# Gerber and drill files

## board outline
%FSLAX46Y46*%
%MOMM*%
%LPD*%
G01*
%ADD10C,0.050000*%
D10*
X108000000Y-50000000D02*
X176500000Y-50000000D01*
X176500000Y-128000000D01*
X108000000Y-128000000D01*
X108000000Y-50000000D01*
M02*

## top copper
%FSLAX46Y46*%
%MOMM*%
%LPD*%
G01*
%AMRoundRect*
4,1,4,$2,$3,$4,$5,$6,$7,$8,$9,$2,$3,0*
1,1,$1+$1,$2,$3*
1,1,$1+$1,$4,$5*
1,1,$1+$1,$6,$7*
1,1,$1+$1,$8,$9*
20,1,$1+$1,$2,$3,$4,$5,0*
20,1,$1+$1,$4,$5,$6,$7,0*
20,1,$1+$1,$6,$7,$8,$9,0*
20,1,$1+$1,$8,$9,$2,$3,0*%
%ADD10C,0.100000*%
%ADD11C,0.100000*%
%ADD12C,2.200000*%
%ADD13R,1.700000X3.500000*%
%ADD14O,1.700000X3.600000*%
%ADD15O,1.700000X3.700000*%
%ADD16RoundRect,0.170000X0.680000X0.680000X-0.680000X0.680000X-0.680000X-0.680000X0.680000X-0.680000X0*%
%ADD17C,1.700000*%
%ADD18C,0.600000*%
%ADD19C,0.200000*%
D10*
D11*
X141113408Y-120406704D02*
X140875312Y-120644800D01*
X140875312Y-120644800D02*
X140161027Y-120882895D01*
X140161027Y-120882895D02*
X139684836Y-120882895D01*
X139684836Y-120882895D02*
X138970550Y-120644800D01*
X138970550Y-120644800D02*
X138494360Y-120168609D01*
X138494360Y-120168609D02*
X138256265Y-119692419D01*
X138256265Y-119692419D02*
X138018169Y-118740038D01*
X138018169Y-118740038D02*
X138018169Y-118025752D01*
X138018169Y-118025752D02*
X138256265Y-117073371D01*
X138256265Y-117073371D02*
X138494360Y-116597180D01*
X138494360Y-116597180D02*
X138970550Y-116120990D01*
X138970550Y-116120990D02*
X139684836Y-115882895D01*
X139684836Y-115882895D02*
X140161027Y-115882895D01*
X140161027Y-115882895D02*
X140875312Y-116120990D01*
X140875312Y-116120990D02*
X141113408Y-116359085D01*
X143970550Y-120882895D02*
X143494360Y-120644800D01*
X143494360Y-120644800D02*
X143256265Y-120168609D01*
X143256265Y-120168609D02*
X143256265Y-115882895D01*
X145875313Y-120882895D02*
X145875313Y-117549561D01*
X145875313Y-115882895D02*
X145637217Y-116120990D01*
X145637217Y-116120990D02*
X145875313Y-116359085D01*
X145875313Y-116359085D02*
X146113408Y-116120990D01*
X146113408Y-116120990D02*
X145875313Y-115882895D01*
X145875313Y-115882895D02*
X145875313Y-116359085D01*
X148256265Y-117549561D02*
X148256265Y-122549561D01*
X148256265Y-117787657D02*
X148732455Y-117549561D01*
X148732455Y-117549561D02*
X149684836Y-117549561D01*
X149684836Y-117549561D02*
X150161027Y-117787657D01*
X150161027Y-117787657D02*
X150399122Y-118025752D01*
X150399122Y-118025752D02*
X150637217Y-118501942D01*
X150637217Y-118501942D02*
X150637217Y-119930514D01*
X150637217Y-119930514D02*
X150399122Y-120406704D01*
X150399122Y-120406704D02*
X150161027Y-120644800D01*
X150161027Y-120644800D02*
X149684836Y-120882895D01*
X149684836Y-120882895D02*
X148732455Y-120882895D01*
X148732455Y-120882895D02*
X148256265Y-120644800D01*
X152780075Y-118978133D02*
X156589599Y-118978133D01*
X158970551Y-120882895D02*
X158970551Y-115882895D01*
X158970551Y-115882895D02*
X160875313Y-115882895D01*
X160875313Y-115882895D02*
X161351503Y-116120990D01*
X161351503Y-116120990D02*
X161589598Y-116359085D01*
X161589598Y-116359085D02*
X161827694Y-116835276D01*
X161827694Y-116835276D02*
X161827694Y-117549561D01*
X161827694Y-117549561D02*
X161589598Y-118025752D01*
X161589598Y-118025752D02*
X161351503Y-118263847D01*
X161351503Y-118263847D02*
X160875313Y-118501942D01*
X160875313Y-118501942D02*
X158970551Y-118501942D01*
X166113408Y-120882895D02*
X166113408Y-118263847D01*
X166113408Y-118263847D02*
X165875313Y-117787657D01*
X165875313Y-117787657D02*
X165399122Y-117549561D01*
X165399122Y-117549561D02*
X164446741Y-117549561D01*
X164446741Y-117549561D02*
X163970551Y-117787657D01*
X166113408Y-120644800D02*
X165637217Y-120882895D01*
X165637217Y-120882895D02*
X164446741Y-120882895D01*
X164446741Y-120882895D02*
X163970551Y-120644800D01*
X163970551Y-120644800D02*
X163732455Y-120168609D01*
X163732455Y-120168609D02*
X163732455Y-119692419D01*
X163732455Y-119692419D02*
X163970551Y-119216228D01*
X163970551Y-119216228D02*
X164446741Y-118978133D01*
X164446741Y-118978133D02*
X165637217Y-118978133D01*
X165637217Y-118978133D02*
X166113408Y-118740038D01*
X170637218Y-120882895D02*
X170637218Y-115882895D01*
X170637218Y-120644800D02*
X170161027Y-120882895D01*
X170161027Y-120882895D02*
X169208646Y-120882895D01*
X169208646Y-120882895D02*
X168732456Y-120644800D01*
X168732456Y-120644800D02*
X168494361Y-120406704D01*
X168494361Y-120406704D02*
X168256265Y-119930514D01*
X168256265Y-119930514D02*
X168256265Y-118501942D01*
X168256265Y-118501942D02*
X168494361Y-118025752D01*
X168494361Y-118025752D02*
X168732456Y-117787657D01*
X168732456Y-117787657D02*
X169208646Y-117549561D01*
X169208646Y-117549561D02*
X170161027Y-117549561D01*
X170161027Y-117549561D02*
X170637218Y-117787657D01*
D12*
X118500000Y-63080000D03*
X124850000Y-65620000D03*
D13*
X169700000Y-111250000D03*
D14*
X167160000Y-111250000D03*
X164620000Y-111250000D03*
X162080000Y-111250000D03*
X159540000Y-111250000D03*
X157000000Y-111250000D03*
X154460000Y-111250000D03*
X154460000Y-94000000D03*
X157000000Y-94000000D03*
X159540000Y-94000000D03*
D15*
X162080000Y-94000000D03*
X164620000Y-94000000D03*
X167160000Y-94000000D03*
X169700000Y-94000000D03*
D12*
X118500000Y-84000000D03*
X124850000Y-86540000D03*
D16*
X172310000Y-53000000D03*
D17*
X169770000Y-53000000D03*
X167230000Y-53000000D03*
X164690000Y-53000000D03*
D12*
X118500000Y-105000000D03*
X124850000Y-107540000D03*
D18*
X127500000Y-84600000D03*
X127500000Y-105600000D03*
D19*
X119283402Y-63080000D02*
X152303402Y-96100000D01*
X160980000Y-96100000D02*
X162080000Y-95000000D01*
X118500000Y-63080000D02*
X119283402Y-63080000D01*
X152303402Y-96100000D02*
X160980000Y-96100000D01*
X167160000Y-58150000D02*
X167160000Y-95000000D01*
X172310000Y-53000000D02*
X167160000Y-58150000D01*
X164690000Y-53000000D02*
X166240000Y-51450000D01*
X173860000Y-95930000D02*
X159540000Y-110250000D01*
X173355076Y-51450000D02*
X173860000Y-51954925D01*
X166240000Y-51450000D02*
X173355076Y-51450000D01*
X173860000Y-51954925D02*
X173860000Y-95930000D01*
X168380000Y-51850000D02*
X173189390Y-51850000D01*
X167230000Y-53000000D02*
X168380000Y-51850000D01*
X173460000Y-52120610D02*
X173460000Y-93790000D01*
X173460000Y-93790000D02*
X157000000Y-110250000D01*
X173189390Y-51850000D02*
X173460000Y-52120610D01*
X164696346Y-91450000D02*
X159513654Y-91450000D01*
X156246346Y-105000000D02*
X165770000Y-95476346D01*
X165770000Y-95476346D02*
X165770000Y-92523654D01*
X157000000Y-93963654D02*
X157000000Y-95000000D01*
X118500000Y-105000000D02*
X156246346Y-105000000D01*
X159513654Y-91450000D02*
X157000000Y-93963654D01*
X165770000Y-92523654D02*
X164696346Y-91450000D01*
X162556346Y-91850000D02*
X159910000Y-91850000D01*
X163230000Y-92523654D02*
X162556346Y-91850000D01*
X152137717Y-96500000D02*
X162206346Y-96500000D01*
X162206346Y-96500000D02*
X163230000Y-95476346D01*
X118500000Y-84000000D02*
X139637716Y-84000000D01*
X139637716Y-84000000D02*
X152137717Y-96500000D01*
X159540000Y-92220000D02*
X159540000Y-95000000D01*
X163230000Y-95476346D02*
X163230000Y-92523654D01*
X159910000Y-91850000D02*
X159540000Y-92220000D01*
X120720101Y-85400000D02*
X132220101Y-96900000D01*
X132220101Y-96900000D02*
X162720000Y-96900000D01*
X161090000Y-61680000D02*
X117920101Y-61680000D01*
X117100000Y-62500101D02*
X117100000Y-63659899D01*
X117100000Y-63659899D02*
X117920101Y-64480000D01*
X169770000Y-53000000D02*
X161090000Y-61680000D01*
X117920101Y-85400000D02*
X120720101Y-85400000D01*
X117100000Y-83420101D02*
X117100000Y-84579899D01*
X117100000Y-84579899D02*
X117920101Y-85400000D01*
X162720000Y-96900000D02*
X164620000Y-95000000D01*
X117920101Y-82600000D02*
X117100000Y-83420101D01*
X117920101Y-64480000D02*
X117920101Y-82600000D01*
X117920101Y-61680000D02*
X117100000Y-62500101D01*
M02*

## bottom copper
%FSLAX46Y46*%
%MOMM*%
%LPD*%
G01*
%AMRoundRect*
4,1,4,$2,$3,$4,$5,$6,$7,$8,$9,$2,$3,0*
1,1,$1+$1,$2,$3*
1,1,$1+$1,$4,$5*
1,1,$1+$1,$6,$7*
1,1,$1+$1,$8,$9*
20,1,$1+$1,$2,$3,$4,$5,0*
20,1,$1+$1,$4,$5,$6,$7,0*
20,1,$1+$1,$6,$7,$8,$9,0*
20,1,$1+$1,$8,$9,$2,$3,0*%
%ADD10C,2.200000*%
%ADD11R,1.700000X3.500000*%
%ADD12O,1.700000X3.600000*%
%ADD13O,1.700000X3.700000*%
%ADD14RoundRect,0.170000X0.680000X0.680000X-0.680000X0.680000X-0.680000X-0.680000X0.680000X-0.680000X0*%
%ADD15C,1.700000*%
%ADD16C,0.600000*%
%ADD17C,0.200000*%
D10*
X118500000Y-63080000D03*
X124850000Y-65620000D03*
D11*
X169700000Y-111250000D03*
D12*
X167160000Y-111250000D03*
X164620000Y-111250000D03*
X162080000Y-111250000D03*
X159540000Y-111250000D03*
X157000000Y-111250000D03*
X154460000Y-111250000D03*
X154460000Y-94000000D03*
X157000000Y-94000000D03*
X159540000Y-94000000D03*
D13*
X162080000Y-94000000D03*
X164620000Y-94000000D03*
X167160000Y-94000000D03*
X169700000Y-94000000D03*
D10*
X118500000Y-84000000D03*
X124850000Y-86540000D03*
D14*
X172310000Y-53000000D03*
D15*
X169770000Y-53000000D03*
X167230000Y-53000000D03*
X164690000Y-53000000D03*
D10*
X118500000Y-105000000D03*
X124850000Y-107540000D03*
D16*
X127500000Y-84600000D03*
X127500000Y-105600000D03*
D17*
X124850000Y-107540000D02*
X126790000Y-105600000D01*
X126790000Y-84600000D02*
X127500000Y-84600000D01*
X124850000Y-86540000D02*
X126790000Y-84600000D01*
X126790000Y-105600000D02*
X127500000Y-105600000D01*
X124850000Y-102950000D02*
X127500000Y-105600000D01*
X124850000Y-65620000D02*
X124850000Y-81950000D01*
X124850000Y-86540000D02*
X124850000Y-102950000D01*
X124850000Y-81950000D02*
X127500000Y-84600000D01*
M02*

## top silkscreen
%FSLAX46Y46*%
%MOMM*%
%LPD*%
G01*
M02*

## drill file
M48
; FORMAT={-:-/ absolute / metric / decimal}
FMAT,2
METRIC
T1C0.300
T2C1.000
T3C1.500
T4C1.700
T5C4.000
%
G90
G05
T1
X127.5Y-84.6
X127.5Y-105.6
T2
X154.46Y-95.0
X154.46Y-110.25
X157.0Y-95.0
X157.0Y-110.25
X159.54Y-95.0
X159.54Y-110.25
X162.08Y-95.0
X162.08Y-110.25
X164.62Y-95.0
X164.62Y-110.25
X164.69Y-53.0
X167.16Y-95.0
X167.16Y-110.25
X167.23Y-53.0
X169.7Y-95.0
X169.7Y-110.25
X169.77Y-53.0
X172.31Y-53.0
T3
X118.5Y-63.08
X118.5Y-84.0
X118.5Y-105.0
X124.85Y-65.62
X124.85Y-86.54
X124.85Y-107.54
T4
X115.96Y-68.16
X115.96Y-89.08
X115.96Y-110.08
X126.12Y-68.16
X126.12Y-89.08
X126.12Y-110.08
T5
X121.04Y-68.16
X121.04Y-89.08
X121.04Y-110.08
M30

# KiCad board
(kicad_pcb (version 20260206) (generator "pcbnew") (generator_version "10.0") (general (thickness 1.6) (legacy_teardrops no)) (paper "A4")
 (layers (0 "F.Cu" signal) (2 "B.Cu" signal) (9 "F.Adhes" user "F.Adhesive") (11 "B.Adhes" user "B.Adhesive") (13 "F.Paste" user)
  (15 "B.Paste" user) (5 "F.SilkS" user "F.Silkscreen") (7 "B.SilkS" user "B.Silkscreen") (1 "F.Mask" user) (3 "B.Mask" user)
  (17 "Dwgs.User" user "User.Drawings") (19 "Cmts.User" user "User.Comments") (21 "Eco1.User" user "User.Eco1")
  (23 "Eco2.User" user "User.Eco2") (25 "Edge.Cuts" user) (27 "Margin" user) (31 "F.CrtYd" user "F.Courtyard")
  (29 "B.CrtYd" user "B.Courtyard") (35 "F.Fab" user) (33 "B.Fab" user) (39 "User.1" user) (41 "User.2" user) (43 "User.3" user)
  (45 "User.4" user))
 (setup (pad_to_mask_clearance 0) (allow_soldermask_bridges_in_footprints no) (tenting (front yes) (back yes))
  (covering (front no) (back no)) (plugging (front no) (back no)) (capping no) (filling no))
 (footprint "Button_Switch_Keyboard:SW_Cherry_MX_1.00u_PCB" (layer "B.Cu") (at 118.5 63.08 180)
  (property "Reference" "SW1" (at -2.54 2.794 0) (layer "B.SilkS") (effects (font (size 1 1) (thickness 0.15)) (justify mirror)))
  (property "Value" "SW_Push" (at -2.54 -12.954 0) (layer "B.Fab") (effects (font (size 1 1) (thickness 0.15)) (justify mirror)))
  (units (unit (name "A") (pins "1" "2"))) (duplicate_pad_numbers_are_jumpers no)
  (pad "" np_thru_hole circle (at -7.62 -5.08 180) (size 1.7 1.7) (drill 1.7) (layers "*.Cu" "*.Mask"))
  (pad "" np_thru_hole circle (at -2.54 -5.08 180) (size 4 4) (drill 4) (layers "*.Cu" "*.Mask"))
  (pad "" np_thru_hole circle (at 2.54 -5.08 180) (size 1.7 1.7) (drill 1.7) (layers "*.Cu" "*.Mask"))
  (pad "1" thru_hole circle (at 0 0 180) (size 2.2 2.2) (drill 1.5) (layers "*.Cu" "*.Mask") (remove_unused_layers no)
   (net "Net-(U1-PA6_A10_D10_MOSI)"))
  (pad "2" thru_hole circle (at -6.35 -2.54 180) (size 2.2 2.2) (drill 1.5) (layers "*.Cu" "*.Mask") (remove_unused_layers no) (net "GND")))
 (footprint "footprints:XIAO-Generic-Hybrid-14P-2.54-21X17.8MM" (layer "B.Cu") (at 162.08 102.625 90)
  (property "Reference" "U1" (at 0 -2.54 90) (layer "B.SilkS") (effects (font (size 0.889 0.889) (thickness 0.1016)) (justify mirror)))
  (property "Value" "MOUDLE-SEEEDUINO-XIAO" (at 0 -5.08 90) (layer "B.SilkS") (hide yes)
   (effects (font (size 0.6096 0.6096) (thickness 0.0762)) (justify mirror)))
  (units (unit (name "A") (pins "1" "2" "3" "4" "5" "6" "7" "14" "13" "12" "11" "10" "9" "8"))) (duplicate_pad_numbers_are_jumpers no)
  (pad "1" thru_hole rect (at -7.625 7.62 90) (size 3.5 1.7) (drill 1 (offset -1 0)) (layers "*.Cu" "*.Mask") (remove_unused_layers no)
   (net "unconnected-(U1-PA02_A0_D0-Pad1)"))
  (pad "2" thru_hole oval (at -7.625 5.08 90) (size 3.6 1.7) (drill 1 (offset -1 0)) (layers "*.Cu" "*.Mask") (remove_unused_layers no)
   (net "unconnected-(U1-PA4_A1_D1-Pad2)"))
  (pad "3" thru_hole oval (at -7.625 2.54 90) (size 3.6 1.7) (drill 1 (offset -1 0)) (layers "*.Cu" "*.Mask") (remove_unused_layers no)
   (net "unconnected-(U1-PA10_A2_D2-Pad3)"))
  (pad "4" thru_hole oval (at -7.625 0 90) (size 3.6 1.7) (drill 1 (offset -1 0)) (layers "*.Cu" "*.Mask") (remove_unused_layers no)
   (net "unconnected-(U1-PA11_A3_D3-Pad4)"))
  (pad "5" thru_hole oval (at -7.625 -2.54 90) (size 3.6 1.7) (drill 1 (offset -1 0)) (layers "*.Cu" "*.Mask") (remove_unused_layers no)
   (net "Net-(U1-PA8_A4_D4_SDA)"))
  (pad "6" thru_hole oval (at -7.625 -5.08 270) (size 3.6 1.7) (drill 1 (offset 1 0)) (layers "*.Cu" "*.Mask") (remove_unused_layers no)
   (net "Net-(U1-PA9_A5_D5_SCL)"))
  (pad "7" thru_hole oval (at -7.625 -7.62 90) (size 3.6 1.7) (drill 1 (offset -1 0)) (layers "*.Cu" "*.Mask") (remove_unused_layers no)
   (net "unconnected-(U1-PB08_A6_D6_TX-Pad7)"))
  (pad "8" thru_hole oval (at 7.625 -7.62 90) (size 3.6 1.7) (drill 1 (offset 1 0)) (layers "*.Cu" "*.Mask") (remove_unused_layers no)
   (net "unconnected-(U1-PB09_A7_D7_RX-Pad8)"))
  (pad "9" thru_hole oval (at 7.625 -5.08 90) (size 3.6 1.7) (drill 1 (offset 1 0)) (layers "*.Cu" "*.Mask") (remove_unused_layers no)
   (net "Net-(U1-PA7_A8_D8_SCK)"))
  (pad "10" thru_hole oval (at 7.625 -2.54 90) (size 3.6 1.7) (drill 1 (offset 1 0)) (layers "*.Cu" "*.Mask") (remove_unused_layers no)
   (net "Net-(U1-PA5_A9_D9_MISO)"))
  (pad "11" thru_hole oval (at 7.625 0 90) (size 3.7 1.7) (drill 1 (offset 1 0)) (layers "*.Cu" "*.Mask") (remove_unused_layers no)
   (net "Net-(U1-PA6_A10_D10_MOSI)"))
  (pad "12" thru_hole oval (at 7.625 2.54 90) (size 3.7 1.7) (drill 1 (offset 1 0)) (layers "*.Cu" "*.Mask") (remove_unused_layers no)
   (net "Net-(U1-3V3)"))
  (pad "13" thru_hole oval (at 7.625 5.08 90) (size 3.7 1.7) (drill 1 (offset 1 0)) (layers "*.Cu" "*.Mask") (remove_unused_layers no)
   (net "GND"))
  (pad "14" thru_hole oval (at 7.625 7.62 90) (size 3.7 1.7) (drill 1 (offset 1 0)) (layers "*.Cu" "*.Mask") (remove_unused_layers no)
   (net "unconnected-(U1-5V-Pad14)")))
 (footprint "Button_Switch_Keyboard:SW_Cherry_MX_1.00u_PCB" (layer "B.Cu") (at 118.5 84 180)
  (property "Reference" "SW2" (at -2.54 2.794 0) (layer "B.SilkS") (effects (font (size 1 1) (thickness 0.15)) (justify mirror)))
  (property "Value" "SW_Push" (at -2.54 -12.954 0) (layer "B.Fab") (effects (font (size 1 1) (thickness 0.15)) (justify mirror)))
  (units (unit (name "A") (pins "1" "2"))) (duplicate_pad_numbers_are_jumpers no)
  (pad "" np_thru_hole circle (at -7.62 -5.08 180) (size 1.7 1.7) (drill 1.7) (layers "*.Cu" "*.Mask"))
  (pad "" np_thru_hole circle (at -2.54 -5.08 180) (size 4 4) (drill 4) (layers "*.Cu" "*.Mask"))
  (pad "" np_thru_hole circle (at 2.54 -5.08 180) (size 1.7 1.7) (drill 1.7) (layers "*.Cu" "*.Mask"))
  (pad "1" thru_hole circle (at 0 0 180) (size 2.2 2.2) (drill 1.5) (layers "*.Cu" "*.Mask") (remove_unused_layers no)
   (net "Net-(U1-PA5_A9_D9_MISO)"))
  (pad "2" thru_hole circle (at -6.35 -2.54 180) (size 2.2 2.2) (drill 1.5) (layers "*.Cu" "*.Mask") (remove_unused_layers no) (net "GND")))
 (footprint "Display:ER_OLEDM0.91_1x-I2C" (layer "B.Cu") (at 172.31 53 180)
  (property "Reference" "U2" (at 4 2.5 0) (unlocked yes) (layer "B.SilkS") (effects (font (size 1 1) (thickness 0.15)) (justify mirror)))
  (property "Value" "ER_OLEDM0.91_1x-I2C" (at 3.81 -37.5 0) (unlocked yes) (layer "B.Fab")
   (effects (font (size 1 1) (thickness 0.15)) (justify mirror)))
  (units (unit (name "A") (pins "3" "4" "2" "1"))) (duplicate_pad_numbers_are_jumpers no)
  (pad "1" thru_hole roundrect (at 0 0 180) (size 1.7 1.7) (drill 1) (layers "*.Cu" "*.Mask") (remove_unused_layers no)
   (roundrect_rratio 0.1) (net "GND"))
  (pad "2" thru_hole circle (at 2.54 0 180) (size 1.7 1.7) (drill 1) (layers "*.Cu" "*.Mask") (remove_unused_layers no) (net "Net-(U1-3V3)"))
  (pad "3" thru_hole circle (at 5.08 0 180) (size 1.7 1.7) (drill 1) (layers "*.Cu" "*.Mask") (remove_unused_layers no)
   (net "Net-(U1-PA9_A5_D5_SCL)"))
  (pad "4" thru_hole circle (at 7.62 0 180) (size 1.7 1.7) (drill 1) (layers "*.Cu" "*.Mask") (remove_unused_layers no)
   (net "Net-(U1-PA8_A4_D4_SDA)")))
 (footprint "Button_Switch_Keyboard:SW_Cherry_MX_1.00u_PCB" (layer "B.Cu") (at 118.5 105 180)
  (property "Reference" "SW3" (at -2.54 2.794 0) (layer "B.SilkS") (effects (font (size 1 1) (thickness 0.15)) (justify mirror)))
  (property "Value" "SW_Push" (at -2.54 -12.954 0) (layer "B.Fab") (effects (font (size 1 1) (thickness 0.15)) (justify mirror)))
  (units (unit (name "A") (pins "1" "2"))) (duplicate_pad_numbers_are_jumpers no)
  (pad "" np_thru_hole circle (at -7.62 -5.08 180) (size 1.7 1.7) (drill 1.7) (layers "*.Cu" "*.Mask"))
  (pad "" np_thru_hole circle (at -2.54 -5.08 180) (size 4 4) (drill 4) (layers "*.Cu" "*.Mask"))
  (pad "" np_thru_hole circle (at 2.54 -5.08 180) (size 1.7 1.7) (drill 1.7) (layers "*.Cu" "*.Mask"))
  (pad "1" thru_hole circle (at 0 0 180) (size 2.2 2.2) (drill 1.5) (layers "*.Cu" "*.Mask") (remove_unused_layers no)
   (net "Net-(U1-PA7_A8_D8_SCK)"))
  (pad "2" thru_hole circle (at -6.35 -2.54 180) (size 2.2 2.2) (drill 1.5) (layers "*.Cu" "*.Mask") (remove_unused_layers no) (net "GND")))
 (gr_rect (start 108 50) (end 176.5 128) (stroke (width 0.05) (type solid)) (fill no) (layer "Edge.Cuts"))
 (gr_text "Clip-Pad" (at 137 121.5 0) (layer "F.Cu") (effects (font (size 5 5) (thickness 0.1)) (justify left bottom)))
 (segment (start 119.283402 63.08) (end 152.303402 96.1) (width 0.2) (layer "F.Cu") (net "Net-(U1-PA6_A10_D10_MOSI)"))
 (segment (start 160.98 96.1) (end 162.08 95) (width 0.2) (layer "F.Cu") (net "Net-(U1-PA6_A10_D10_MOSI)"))
 (segment (start 118.5 63.08) (end 119.283402 63.08) (width 0.2) (layer "F.Cu") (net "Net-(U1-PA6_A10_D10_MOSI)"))
 (segment (start 152.303402 96.1) (end 160.98 96.1) (width 0.2) (layer "F.Cu") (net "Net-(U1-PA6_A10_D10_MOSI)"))
 (segment (start 167.16 58.15) (end 167.16 95) (width 0.2) (layer "F.Cu") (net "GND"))
 (segment (start 172.31 53) (end 167.16 58.15) (width 0.2) (layer "F.Cu") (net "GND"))
 (via (at 127.5 84.6) (size 0.6) (drill 0.3) (layers "F.Cu" "B.Cu") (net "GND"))
 (via (at 127.5 105.6) (size 0.6) (drill 0.3) (layers "F.Cu" "B.Cu") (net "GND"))
 (segment (start 124.85 107.54) (end 126.79 105.6) (width 0.2) (layer "B.Cu") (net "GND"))
 (segment (start 126.79 84.6) (end 127.5 84.6) (width 0.2) (layer "B.Cu") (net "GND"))
 (segment (start 124.85 86.54) (end 126.79 84.6) (width 0.2) (layer "B.Cu") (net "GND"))
 (segment (start 126.79 105.6) (end 127.5 105.6) (width 0.2) (layer "B.Cu") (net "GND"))
 (segment (start 124.85 102.95) (end 127.5 105.6) (width 0.2) (layer "B.Cu") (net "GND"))
 (segment (start 124.85 65.62) (end 124.85 81.95) (width 0.2) (layer "B.Cu") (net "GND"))
 (segment (start 124.85 86.54) (end 124.85 102.95) (width 0.2) (layer "B.Cu") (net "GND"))
 (segment (start 124.85 81.95) (end 127.5 84.6) (width 0.2) (layer "B.Cu") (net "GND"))
 (segment (start 164.69 53) (end 166.24 51.45) (width 0.2) (layer "F.Cu") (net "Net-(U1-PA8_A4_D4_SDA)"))
 (segment (start 173.86 95.93) (end 159.54 110.25) (width 0.2) (layer "F.Cu") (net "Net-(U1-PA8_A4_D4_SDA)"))
 (segment (start 173.355076 51.45) (end 173.86 51.954925) (width 0.2) (layer "F.Cu") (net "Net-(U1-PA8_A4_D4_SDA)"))
 (segment (start 166.24 51.45) (end 173.355076 51.45) (width 0.2) (layer "F.Cu") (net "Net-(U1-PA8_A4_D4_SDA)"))
 (segment (start 173.86 51.954925) (end 173.86 95.93) (width 0.2) (layer "F.Cu") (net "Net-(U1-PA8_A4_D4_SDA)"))
 (segment (start 168.38 51.85) (end 173.18939 51.85) (width 0.2) (layer "F.Cu") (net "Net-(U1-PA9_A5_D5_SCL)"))
 (segment (start 167.23 53) (end 168.38 51.85) (width 0.2) (layer "F.Cu") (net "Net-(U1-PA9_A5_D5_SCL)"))
 (segment (start 173.46 52.12061) (end 173.46 93.79) (width 0.2) (layer "F.Cu") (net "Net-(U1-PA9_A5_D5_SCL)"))
 (segment (start 173.46 93.79) (end 157 110.25) (width 0.2) (layer "F.Cu") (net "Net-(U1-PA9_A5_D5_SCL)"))
 (segment (start 173.18939 51.85) (end 173.46 52.12061) (width 0.2) (layer "F.Cu") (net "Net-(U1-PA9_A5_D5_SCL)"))
 (segment (start 164.696346 91.45) (end 159.513654 91.45) (width 0.2) (layer "F.Cu") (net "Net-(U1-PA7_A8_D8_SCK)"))
 (segment (start 156.246346 105) (end 165.77 95.476346) (width 0.2) (layer "F.Cu") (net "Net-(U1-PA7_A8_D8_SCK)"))
 (segment (start 165.77 95.476346) (end 165.77 92.523654) (width 0.2) (layer "F.Cu") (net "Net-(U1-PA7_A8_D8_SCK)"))
 (segment (start 157 93.963654) (end 157 95) (width 0.2) (layer "F.Cu") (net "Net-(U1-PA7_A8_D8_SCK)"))
 (segment (start 118.5 105) (end 156.246346 105) (width 0.2) (layer "F.Cu") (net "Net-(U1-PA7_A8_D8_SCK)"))
 (segment (start 159.513654 91.45) (end 157 93.963654) (width 0.2) (layer "F.Cu") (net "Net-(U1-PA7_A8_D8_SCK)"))
 (segment (start 165.77 92.523654) (end 164.696346 91.45) (width 0.2) (layer "F.Cu") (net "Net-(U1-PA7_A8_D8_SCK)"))
 (segment (start 162.556346 91.85) (end 159.91 91.85) (width 0.2) (layer "F.Cu") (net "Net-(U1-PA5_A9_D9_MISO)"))
 (segment (start 163.23 92.523654) (end 162.556346 91.85) (width 0.2) (layer "F.Cu") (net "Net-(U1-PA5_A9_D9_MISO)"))
 (segment (start 152.137717 96.5) (end 162.206346 96.5) (width 0.2) (layer "F.Cu") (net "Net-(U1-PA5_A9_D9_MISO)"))
 (segment (start 162.206346 96.5) (end 163.23 95.476346) (width 0.2) (layer "F.Cu") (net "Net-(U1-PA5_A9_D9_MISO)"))
 (segment (start 118.5 84) (end 139.637716 84) (width 0.2) (layer "F.Cu") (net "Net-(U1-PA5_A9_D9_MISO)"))
 (segment (start 139.637716 84) (end 152.137717 96.5) (width 0.2) (layer "F.Cu") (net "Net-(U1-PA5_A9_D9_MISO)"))
 (segment (start 159.54 92.22) (end 159.54 95) (width 0.2) (layer "F.Cu") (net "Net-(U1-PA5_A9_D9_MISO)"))
 (segment (start 163.23 95.476346) (end 163.23 92.523654) (width 0.2) (layer "F.Cu") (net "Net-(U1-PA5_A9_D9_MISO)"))
 (segment (start 159.91 91.85) (end 159.54 92.22) (width 0.2) (layer "F.Cu") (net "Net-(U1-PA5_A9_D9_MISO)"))
 (segment (start 120.720101 85.4) (end 132.220101 96.9) (width 0.2) (layer "F.Cu") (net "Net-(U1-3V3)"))
 (segment (start 132.220101 96.9) (end 162.72 96.9) (width 0.2) (layer "F.Cu") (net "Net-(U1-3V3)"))
 (segment (start 161.09 61.68) (end 117.920101 61.68) (width 0.2) (layer "F.Cu") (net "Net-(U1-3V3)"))
 (segment (start 117.1 62.500101) (end 117.1 63.659899) (width 0.2) (layer "F.Cu") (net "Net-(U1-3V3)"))
 (segment (start 117.1 63.659899) (end 117.920101 64.48) (width 0.2) (layer "F.Cu") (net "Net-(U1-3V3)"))
 (segment (start 169.77 53) (end 161.09 61.68) (width 0.2) (layer "F.Cu") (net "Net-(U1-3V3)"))
 (segment (start 117.920101 85.4) (end 120.720101 85.4) (width 0.2) (layer "F.Cu") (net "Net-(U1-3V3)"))
 (segment (start 117.1 83.420101) (end 117.1 84.579899) (width 0.2) (layer "F.Cu") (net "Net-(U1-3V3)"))
 (segment (start 117.1 84.579899) (end 117.920101 85.4) (width 0.2) (layer "F.Cu") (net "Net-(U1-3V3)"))
 (segment (start 162.72 96.9) (end 164.62 95) (width 0.2) (layer "F.Cu") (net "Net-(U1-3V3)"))
 (segment (start 117.920101 82.6) (end 117.1 83.420101) (width 0.2) (layer "F.Cu") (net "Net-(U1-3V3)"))
 (segment (start 117.920101 64.48) (end 117.920101 82.6) (width 0.2) (layer "F.Cu") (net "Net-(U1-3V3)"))
 (segment (start 117.920101 61.68) (end 117.1 62.500101) (width 0.2) (layer "F.Cu") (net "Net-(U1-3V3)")))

